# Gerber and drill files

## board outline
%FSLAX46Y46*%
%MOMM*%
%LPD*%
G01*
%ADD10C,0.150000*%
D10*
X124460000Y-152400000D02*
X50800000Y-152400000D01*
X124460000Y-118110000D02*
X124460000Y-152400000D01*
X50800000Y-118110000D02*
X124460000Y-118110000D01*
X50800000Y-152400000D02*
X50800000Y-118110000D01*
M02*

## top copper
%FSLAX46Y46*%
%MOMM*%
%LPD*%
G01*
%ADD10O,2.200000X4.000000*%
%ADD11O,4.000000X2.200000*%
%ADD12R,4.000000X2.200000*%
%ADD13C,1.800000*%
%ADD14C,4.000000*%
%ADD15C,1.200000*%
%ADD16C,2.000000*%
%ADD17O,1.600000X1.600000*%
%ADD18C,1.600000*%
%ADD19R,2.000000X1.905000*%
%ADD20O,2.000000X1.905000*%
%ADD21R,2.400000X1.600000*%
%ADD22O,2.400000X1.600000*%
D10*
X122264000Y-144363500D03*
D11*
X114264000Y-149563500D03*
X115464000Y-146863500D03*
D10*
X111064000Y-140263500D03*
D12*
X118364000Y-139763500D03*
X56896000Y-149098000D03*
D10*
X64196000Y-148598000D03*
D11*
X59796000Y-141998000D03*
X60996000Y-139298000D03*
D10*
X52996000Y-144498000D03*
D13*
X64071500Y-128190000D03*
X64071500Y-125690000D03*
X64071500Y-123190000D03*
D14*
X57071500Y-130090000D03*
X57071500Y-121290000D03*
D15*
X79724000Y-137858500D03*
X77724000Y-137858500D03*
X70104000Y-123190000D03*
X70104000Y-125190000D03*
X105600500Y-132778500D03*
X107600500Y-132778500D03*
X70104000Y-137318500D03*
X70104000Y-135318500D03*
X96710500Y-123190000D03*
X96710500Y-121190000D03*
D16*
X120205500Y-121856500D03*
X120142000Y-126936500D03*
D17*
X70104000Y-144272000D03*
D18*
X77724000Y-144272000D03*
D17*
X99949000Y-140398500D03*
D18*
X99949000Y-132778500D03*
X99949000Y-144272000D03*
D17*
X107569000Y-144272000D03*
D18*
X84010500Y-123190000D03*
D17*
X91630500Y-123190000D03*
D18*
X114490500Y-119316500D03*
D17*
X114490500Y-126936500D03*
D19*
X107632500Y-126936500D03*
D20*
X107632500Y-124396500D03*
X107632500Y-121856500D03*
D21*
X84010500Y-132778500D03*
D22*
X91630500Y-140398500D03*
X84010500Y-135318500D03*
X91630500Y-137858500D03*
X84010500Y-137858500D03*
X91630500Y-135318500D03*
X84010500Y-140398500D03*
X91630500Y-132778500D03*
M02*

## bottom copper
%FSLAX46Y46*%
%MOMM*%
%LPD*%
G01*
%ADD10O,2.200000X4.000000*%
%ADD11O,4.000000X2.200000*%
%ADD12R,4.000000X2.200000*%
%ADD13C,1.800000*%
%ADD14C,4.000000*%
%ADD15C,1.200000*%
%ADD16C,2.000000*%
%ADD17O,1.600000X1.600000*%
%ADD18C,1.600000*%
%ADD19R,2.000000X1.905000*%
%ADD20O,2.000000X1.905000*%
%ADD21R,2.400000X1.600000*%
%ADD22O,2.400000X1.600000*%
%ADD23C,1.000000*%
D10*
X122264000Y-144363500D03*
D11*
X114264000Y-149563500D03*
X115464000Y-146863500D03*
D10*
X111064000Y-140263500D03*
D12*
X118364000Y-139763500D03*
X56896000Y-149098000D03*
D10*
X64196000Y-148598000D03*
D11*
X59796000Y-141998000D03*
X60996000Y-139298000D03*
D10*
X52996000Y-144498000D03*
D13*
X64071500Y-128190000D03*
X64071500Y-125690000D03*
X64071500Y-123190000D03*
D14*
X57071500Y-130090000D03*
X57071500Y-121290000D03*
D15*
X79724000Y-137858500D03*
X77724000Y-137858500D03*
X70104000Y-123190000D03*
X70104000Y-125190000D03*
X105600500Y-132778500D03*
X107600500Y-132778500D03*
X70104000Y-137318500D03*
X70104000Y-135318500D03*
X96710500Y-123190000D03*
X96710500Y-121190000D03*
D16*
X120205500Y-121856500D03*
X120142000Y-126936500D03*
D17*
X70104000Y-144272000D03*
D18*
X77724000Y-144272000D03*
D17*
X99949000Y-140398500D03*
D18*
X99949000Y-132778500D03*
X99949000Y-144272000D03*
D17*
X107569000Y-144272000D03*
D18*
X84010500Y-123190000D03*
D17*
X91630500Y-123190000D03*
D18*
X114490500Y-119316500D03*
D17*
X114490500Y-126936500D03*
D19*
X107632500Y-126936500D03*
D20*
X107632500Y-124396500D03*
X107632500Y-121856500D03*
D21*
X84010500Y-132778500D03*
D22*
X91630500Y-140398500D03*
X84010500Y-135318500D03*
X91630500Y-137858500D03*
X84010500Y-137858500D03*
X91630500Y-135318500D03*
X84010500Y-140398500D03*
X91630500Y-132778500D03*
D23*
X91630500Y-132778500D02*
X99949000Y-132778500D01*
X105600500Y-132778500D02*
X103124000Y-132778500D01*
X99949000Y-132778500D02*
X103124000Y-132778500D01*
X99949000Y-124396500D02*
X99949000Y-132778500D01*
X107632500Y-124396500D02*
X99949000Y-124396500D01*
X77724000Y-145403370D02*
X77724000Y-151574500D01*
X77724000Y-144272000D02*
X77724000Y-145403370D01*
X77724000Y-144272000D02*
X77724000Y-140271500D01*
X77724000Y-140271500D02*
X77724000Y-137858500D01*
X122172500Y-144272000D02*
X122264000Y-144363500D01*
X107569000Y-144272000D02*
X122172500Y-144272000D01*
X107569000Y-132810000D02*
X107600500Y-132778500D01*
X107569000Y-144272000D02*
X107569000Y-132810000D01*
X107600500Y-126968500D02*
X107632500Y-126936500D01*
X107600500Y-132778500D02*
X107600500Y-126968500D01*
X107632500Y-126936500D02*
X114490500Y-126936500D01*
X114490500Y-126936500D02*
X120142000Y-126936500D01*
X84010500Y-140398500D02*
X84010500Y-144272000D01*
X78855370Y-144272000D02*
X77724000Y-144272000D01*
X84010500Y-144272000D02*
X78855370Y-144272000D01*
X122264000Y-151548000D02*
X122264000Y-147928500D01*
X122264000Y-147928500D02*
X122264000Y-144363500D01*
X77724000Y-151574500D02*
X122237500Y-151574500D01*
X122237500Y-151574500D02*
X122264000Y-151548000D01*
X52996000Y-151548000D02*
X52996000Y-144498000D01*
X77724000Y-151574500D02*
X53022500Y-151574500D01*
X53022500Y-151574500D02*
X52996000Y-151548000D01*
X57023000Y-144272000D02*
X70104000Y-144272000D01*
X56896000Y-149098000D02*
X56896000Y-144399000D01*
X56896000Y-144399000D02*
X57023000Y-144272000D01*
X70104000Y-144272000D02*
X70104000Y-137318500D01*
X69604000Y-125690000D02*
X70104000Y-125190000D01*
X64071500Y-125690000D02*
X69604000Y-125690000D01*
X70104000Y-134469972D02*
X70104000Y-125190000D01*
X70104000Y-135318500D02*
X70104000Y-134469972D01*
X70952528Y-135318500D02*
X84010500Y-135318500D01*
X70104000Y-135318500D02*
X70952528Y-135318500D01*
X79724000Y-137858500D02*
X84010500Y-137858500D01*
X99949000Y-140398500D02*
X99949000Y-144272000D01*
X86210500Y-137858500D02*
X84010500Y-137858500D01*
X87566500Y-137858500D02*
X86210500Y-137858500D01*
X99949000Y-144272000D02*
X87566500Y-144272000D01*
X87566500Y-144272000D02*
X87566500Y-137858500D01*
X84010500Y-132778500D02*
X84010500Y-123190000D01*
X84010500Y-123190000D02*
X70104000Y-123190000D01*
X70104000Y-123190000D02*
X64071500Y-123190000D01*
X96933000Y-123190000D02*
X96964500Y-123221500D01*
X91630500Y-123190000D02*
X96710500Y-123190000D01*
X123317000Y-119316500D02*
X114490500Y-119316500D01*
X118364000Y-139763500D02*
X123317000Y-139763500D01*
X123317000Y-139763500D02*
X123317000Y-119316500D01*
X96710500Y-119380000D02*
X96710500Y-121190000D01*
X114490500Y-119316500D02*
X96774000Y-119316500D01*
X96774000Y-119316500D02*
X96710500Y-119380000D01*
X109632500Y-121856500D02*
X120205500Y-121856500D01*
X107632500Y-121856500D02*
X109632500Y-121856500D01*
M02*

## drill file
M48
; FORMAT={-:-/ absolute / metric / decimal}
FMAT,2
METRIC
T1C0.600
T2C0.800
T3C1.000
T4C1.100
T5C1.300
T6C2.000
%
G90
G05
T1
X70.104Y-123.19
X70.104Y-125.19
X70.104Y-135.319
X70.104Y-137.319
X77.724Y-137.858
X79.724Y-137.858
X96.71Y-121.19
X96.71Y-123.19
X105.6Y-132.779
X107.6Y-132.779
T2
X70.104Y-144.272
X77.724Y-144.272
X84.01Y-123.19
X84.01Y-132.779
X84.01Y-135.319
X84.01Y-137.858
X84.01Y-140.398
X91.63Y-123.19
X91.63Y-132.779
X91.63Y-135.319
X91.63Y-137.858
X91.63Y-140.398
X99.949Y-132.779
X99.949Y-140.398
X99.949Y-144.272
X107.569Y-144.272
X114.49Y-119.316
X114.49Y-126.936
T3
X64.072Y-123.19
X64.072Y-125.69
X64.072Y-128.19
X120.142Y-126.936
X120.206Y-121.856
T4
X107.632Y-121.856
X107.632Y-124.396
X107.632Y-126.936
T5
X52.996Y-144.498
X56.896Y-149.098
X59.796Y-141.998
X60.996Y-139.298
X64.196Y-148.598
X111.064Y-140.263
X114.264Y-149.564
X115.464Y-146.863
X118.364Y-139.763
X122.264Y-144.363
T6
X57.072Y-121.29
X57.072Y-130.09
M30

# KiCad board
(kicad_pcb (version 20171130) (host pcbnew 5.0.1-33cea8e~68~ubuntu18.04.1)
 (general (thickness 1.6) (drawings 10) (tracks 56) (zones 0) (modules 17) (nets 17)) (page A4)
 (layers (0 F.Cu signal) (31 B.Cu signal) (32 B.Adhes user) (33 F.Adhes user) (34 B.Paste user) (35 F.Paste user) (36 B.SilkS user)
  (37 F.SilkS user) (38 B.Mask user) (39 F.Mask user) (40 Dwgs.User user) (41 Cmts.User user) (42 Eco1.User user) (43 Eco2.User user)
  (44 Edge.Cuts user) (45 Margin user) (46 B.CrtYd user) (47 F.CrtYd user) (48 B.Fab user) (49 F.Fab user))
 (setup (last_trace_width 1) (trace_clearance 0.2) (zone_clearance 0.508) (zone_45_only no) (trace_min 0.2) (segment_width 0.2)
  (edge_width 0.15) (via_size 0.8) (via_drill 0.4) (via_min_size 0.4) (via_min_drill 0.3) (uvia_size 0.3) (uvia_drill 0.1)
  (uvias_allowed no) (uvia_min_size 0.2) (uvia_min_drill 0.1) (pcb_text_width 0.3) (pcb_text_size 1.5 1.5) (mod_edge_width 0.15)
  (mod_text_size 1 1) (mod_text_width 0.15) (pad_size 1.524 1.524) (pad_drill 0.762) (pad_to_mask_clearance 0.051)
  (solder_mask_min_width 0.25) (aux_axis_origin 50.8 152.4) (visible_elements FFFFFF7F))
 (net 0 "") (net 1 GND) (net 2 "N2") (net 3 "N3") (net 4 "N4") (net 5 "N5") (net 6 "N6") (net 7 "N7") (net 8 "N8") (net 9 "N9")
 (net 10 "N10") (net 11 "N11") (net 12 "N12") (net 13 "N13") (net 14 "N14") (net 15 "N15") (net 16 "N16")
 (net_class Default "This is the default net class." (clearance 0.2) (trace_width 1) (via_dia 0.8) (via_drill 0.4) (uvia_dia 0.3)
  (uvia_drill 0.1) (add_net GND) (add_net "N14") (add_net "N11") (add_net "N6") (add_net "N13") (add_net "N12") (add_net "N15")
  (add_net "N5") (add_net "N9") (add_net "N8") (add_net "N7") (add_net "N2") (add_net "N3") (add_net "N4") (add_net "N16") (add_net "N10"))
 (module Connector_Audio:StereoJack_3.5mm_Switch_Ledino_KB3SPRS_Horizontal (layer F.Cu) (at 118.364 139.7635 180)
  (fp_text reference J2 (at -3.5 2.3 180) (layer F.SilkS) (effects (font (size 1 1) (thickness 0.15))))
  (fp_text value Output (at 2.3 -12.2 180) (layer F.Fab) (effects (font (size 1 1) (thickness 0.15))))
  (pad S thru_hole oval (at -3.9 -4.6 180) (size 2.2 4) (drill 1.3) (layers *.Cu *.Mask) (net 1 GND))
  (pad R thru_hole oval (at 4.1 -9.8 180) (size 4 2.2) (drill 1.3) (layers *.Cu *.Mask) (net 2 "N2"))
  (pad RN thru_hole oval (at 2.9 -7.1 180) (size 4 2.2) (drill 1.3) (layers *.Cu *.Mask) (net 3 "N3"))
  (pad TN thru_hole oval (at 7.3 -0.5 270) (size 4 2.2) (drill 1.3) (layers *.Cu *.Mask) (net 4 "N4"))
  (pad T thru_hole rect (at 0 0 180) (size 4 2.2) (drill 1.3) (layers *.Cu *.Mask) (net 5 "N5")))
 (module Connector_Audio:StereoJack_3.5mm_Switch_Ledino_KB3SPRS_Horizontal (layer F.Cu) (at 56.896 149.098)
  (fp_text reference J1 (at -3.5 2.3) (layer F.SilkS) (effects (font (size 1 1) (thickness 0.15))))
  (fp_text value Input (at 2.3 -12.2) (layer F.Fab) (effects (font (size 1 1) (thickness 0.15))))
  (pad T thru_hole rect (at 0 0) (size 4 2.2) (drill 1.3) (layers *.Cu *.Mask) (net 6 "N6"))
  (pad TN thru_hole oval (at 7.3 -0.5 90) (size 4 2.2) (drill 1.3) (layers *.Cu *.Mask) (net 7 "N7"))
  (pad RN thru_hole oval (at 2.9 -7.1) (size 4 2.2) (drill 1.3) (layers *.Cu *.Mask) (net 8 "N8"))
  (pad R thru_hole oval (at 4.1 -9.8) (size 4 2.2) (drill 1.3) (layers *.Cu *.Mask) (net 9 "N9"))
  (pad S thru_hole oval (at -3.9 -4.6) (size 2.2 4) (drill 1.3) (layers *.Cu *.Mask) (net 1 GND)))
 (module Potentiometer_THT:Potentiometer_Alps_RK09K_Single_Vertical (layer F.Cu) (at 64.0715 123.19 180)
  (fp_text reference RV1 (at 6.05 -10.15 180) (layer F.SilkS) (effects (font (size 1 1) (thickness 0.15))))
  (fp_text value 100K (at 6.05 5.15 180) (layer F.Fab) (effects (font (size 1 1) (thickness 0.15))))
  (pad 3 thru_hole circle (at 0 -5 180) (size 1.8 1.8) (drill 1) (layers *.Cu *.Mask) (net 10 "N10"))
  (pad 2 thru_hole circle (at 0 -2.5 180) (size 1.8 1.8) (drill 1) (layers *.Cu *.Mask) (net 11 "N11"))
  (pad 1 thru_hole circle (at 0 0 180) (size 1.8 1.8) (drill 1) (layers *.Cu *.Mask) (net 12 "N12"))
  (pad "" np_thru_hole circle (at 7 -6.9 180) (size 4 4) (drill 2) (layers *.Cu *.Mask))
  (pad "" np_thru_hole circle (at 7 1.9 180) (size 4 4) (drill 2) (layers *.Cu *.Mask)))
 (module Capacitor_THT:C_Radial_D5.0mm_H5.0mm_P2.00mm (layer F.Cu) (at 77.724 137.8585)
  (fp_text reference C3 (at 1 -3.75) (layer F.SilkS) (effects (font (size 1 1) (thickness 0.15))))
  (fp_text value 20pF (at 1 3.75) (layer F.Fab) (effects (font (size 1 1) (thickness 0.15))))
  (pad 2 thru_hole circle (at 2 0) (size 1.2 1.2) (drill 0.6) (layers *.Cu *.Mask) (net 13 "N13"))
  (pad 1 thru_hole circle (at 0 0) (size 1.2 1.2) (drill 0.6) (layers *.Cu *.Mask) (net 1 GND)))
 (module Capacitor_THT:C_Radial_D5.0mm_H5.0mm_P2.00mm (layer F.Cu) (at 70.104 123.19 270)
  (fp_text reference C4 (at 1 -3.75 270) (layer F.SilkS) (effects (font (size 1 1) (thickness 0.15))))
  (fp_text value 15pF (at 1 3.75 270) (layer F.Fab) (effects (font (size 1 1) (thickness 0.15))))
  (pad 1 thru_hole circle (at 0 0 270) (size 1.2 1.2) (drill 0.6) (layers *.Cu *.Mask) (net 12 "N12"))
  (pad 2 thru_hole circle (at 2 0 270) (size 1.2 1.2) (drill 0.6) (layers *.Cu *.Mask) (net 11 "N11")))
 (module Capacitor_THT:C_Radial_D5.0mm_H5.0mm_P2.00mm (layer F.Cu) (at 105.6005 132.7785)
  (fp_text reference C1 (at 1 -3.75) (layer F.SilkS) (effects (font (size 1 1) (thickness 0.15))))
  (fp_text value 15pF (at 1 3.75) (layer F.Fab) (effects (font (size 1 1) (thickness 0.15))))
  (pad 1 thru_hole circle (at 0 0) (size 1.2 1.2) (drill 0.6) (layers *.Cu *.Mask) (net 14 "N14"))
  (pad 2 thru_hole circle (at 2 0) (size 1.2 1.2) (drill 0.6) (layers *.Cu *.Mask) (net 1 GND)))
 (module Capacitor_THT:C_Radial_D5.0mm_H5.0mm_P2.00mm (layer F.Cu) (at 70.104 135.3185 270)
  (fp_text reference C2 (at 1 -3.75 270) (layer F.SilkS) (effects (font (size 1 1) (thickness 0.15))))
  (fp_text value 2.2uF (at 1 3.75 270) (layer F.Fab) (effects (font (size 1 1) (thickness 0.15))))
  (pad 2 thru_hole circle (at 2 0 270) (size 1.2 1.2) (drill 0.6) (layers *.Cu *.Mask) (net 6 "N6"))
  (pad 1 thru_hole circle (at 0 0 270) (size 1.2 1.2) (drill 0.6) (layers *.Cu *.Mask) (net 11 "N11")))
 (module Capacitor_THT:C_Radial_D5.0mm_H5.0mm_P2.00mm (layer F.Cu) (at 96.7105 123.19 90)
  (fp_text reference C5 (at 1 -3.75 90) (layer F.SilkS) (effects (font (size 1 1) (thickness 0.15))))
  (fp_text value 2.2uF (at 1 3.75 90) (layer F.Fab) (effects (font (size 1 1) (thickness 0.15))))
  (pad 1 thru_hole circle (at 0 0 90) (size 1.2 1.2) (drill 0.6) (layers *.Cu *.Mask) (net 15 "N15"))
  (pad 2 thru_hole circle (at 2 0 90) (size 1.2 1.2) (drill 0.6) (layers *.Cu *.Mask) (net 5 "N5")))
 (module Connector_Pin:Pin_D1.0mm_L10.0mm (layer F.Cu) (at 120.2055 121.8565)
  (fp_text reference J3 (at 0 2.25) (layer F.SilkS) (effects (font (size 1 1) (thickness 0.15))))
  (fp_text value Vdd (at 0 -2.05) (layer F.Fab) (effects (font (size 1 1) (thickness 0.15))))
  (pad 1 thru_hole circle (at 0 0) (size 2 2) (drill 1) (layers *.Cu *.Mask) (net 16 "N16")))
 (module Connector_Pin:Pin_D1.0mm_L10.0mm (layer F.Cu) (at 120.142 126.9365)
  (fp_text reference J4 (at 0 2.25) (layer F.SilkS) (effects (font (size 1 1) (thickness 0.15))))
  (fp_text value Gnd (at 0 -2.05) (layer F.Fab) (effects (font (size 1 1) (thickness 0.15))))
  (pad 1 thru_hole circle (at 0 0) (size 2 2) (drill 1) (layers *.Cu *.Mask) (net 1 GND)))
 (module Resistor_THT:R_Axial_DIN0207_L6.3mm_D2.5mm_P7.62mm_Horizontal (layer F.Cu) (at 77.724 144.272 180)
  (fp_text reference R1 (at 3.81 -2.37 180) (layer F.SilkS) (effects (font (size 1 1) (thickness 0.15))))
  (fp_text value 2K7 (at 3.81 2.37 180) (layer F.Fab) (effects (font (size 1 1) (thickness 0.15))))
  (pad 2 thru_hole oval (at 7.62 0 180) (size 1.6 1.6) (drill 0.8) (layers *.Cu *.Mask) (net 6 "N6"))
  (pad 1 thru_hole circle (at 0 0 180) (size 1.6 1.6) (drill 0.8) (layers *.Cu *.Mask) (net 1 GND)))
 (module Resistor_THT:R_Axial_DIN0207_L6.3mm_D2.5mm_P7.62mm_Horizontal (layer F.Cu) (at 99.949 132.7785 270)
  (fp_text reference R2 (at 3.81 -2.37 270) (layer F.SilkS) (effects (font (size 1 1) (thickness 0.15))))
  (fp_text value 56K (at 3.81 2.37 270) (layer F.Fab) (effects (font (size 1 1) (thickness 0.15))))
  (pad 2 thru_hole oval (at 7.62 0 270) (size 1.6 1.6) (drill 0.8) (layers *.Cu *.Mask) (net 13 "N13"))
  (pad 1 thru_hole circle (at 0 0 270) (size 1.6 1.6) (drill 0.8) (layers *.Cu *.Mask) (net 14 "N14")))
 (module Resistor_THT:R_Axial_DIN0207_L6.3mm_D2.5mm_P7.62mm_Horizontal (layer F.Cu) (at 99.949 144.272)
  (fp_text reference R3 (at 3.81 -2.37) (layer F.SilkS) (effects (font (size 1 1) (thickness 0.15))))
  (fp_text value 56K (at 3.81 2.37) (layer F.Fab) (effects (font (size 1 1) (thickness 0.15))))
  (pad 1 thru_hole circle (at 0 0) (size 1.6 1.6) (drill 0.8) (layers *.Cu *.Mask) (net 13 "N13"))
  (pad 2 thru_hole oval (at 7.62 0) (size 1.6 1.6) (drill 0.8) (layers *.Cu *.Mask) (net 1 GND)))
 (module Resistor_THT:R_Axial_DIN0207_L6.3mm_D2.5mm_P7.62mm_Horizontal (layer F.Cu) (at 84.0105 123.19)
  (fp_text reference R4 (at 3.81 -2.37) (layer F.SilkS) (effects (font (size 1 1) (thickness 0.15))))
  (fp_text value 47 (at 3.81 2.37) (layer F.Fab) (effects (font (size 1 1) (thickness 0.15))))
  (pad 1 thru_hole circle (at 0 0) (size 1.6 1.6) (drill 0.8) (layers *.Cu *.Mask) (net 12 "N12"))
  (pad 2 thru_hole oval (at 7.62 0) (size 1.6 1.6) (drill 0.8) (layers *.Cu *.Mask) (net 15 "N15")))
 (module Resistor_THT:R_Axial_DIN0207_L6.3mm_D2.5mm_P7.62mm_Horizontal (layer F.Cu) (at 114.4905 119.3165 270)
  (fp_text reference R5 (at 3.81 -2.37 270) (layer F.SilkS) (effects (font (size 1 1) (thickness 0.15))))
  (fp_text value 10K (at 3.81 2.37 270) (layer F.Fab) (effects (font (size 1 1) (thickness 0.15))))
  (pad 1 thru_hole circle (at 0 0 270) (size 1.6 1.6) (drill 0.8) (layers *.Cu *.Mask) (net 5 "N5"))
  (pad 2 thru_hole oval (at 7.62 0 270) (size 1.6 1.6) (drill 0.8) (layers *.Cu *.Mask) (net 1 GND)))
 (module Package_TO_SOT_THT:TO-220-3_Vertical (layer F.Cu) (at 107.6325 126.9365 90)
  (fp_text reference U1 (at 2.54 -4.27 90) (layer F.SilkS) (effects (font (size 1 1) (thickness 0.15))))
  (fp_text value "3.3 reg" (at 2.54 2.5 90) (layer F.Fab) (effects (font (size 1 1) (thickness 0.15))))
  (pad 1 thru_hole rect (at 0 0 90) (size 1.905 2) (drill 1.1) (layers *.Cu *.Mask) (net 1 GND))
  (pad 2 thru_hole oval (at 2.54 0 90) (size 1.905 2) (drill 1.1) (layers *.Cu *.Mask) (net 14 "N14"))
  (pad 3 thru_hole oval (at 5.08 0 90) (size 1.905 2) (drill 1.1) (layers *.Cu *.Mask) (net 16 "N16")))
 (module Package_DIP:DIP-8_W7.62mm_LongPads (layer F.Cu) (at 84.0105 132.7785)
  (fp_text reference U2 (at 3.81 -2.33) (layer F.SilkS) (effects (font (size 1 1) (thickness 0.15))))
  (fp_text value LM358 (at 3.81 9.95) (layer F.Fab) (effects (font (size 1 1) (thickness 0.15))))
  (pad 1 thru_hole rect (at 0 0) (size 2.4 1.6) (drill 0.8) (layers *.Cu *.Mask) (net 12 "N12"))
  (pad 5 thru_hole oval (at 7.62 7.62) (size 2.4 1.6) (drill 0.8) (layers *.Cu *.Mask))
  (pad 2 thru_hole oval (at 0 2.54) (size 2.4 1.6) (drill 0.8) (layers *.Cu *.Mask) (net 11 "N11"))
  (pad 6 thru_hole oval (at 7.62 5.08) (size 2.4 1.6) (drill 0.8) (layers *.Cu *.Mask))
  (pad 3 thru_hole oval (at 0 5.08) (size 2.4 1.6) (drill 0.8) (layers *.Cu *.Mask) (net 13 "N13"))
  (pad 7 thru_hole oval (at 7.62 2.54) (size 2.4 1.6) (drill 0.8) (layers *.Cu *.Mask))
  (pad 4 thru_hole oval (at 0 7.62) (size 2.4 1.6) (drill 0.8) (layers *.Cu *.Mask) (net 1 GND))
  (pad 8 thru_hole oval (at 7.62 0) (size 2.4 1.6) (drill 0.8) (layers *.Cu *.Mask) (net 14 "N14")))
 (gr_line (start 124.46 152.4) (end 50.8 152.4) (layer Edge.Cuts) (width 0.15))
 (gr_line (start 124.46 118.11) (end 124.46 152.4) (layer Edge.Cuts) (width 0.15))
 (gr_line (start 50.8 118.11) (end 124.46 118.11) (layer Edge.Cuts) (width 0.15))
 (gr_line (start 50.8 152.4) (end 50.8 118.11) (layer Edge.Cuts) (width 0.15))
 (segment (start 91.6305 132.7785) (end 99.949 132.7785) (width 1) (layer B.Cu) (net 14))
 (segment (start 105.6005 132.7785) (end 103.124 132.7785) (width 1) (layer B.Cu) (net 14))
 (segment (start 99.949 132.7785) (end 103.124 132.7785) (width 1) (layer B.Cu) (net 14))
 (segment (start 99.949 124.3965) (end 99.949 132.7785) (width 1) (layer B.Cu) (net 14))
 (segment (start 107.6325 124.3965) (end 99.949 124.3965) (width 1) (layer B.Cu) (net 14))
 (segment (start 77.724 145.40337) (end 77.724 151.5745) (width 1) (layer B.Cu) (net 1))
 (segment (start 77.724 144.272) (end 77.724 145.40337) (width 1) (layer B.Cu) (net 1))
 (segment (start 77.724 144.272) (end 77.724 140.2715) (width 1) (layer B.Cu) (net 1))
 (segment (start 77.724 140.2715) (end 77.724 137.8585) (width 1) (layer B.Cu) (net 1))
 (segment (start 122.1725 144.272) (end 122.264 144.3635) (width 1) (layer B.Cu) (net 1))
 (segment (start 107.569 144.272) (end 122.1725 144.272) (width 1) (layer B.Cu) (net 1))
 (segment (start 107.569 132.81) (end 107.6005 132.7785) (width 1) (layer B.Cu) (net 1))
 (segment (start 107.569 144.272) (end 107.569 132.81) (width 1) (layer B.Cu) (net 1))
 (segment (start 107.6005 126.9685) (end 107.6325 126.9365) (width 1) (layer B.Cu) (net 1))
 (segment (start 107.6005 132.7785) (end 107.6005 126.9685) (width 1) (layer B.Cu) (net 1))
 (segment (start 107.6325 126.9365) (end 114.4905 126.9365) (width 1) (layer B.Cu) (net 1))
 (segment (start 114.4905 126.9365) (end 120.142 126.9365) (width 1) (layer B.Cu) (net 1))
 (segment (start 84.0105 140.3985) (end 84.0105 144.272) (width 1) (layer B.Cu) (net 1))
 (segment (start 78.85537 144.272) (end 77.724 144.272) (width 1) (layer B.Cu) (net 1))
 (segment (start 84.0105 144.272) (end 78.85537 144.272) (width 1) (layer B.Cu) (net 1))
 (segment (start 122.264 151.548) (end 122.264 147.9285) (width 1) (layer B.Cu) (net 1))
 (segment (start 122.264 147.9285) (end 122.264 144.3635) (width 1) (layer B.Cu) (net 1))
 (segment (start 77.724 151.5745) (end 122.2375 151.5745) (width 1) (layer B.Cu) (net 1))
 (segment (start 122.2375 151.5745) (end 122.264 151.548) (width 1) (layer B.Cu) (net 1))
 (segment (start 52.996 151.548) (end 52.996 144.498) (width 1) (layer B.Cu) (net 1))
 (segment (start 77.724 151.5745) (end 53.0225 151.5745) (width 1) (layer B.Cu) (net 1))
 (segment (start 53.0225 151.5745) (end 52.996 151.548) (width 1) (layer B.Cu) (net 1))
 (segment (start 57.023 144.272) (end 70.104 144.272) (width 1) (layer B.Cu) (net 6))
 (segment (start 56.896 149.098) (end 56.896 144.399) (width 1) (layer B.Cu) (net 6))
 (segment (start 56.896 144.399) (end 57.023 144.272) (width 1) (layer B.Cu) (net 6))
 (segment (start 70.104 144.272) (end 70.104 137.3185) (width 1) (layer B.Cu) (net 6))
 (segment (start 69.604 125.69) (end 70.104 125.19) (width 1) (layer B.Cu) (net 11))
 (segment (start 64.0715 125.69) (end 69.604 125.69) (width 1) (layer B.Cu) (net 11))
 (segment (start 70.104 134.469972) (end 70.104 125.19) (width 1) (layer B.Cu) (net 11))
 (segment (start 70.104 135.3185) (end 70.104 134.469972) (width 1) (layer B.Cu) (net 11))
 (segment (start 70.952528 135.3185) (end 84.0105 135.3185) (width 1) (layer B.Cu) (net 11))
 (segment (start 70.104 135.3185) (end 70.952528 135.3185) (width 1) (layer B.Cu) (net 11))
 (segment (start 79.724 137.8585) (end 84.0105 137.8585) (width 1) (layer B.Cu) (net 13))
 (segment (start 99.949 140.3985) (end 99.949 144.272) (width 1) (layer B.Cu) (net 13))
 (segment (start 86.2105 137.8585) (end 84.0105 137.8585) (width 1) (layer B.Cu) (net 13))
 (segment (start 87.5665 137.8585) (end 86.2105 137.8585) (width 1) (layer B.Cu) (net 13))
 (segment (start 99.949 144.272) (end 87.5665 144.272) (width 1) (layer B.Cu) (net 13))
 (segment (start 87.5665 144.272) (end 87.5665 137.8585) (width 1) (layer B.Cu) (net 13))
 (segment (start 84.0105 132.7785) (end 84.0105 123.19) (width 1) (layer B.Cu) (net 12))
 (segment (start 84.0105 123.19) (end 70.104 123.19) (width 1) (layer B.Cu) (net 12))
 (segment (start 70.104 123.19) (end 64.0715 123.19) (width 1) (layer B.Cu) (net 12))
 (segment (start 96.933 123.19) (end 96.9645 123.2215) (width 1) (layer B.Cu) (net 15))
 (segment (start 91.6305 123.19) (end 96.7105 123.19) (width 1) (layer B.Cu) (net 15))
 (segment (start 123.317 119.3165) (end 114.4905 119.3165) (width 1) (layer B.Cu) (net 5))
 (segment (start 118.364 139.7635) (end 123.317 139.7635) (width 1) (layer B.Cu) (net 5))
 (segment (start 123.317 139.7635) (end 123.317 119.3165) (width 1) (layer B.Cu) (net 5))
 (segment (start 96.7105 119.38) (end 96.7105 121.19) (width 1) (layer B.Cu) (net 5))
 (segment (start 114.4905 119.3165) (end 96.774 119.3165) (width 1) (layer B.Cu) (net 5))
 (segment (start 96.774 119.3165) (end 96.7105 119.38) (width 1) (layer B.Cu) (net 5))
 (segment (start 109.6325 121.8565) (end 120.2055 121.8565) (width 1) (layer B.Cu) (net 16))
 (segment (start 107.6325 121.8565) (end 109.6325 121.8565) (width 1) (layer B.Cu) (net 16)))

